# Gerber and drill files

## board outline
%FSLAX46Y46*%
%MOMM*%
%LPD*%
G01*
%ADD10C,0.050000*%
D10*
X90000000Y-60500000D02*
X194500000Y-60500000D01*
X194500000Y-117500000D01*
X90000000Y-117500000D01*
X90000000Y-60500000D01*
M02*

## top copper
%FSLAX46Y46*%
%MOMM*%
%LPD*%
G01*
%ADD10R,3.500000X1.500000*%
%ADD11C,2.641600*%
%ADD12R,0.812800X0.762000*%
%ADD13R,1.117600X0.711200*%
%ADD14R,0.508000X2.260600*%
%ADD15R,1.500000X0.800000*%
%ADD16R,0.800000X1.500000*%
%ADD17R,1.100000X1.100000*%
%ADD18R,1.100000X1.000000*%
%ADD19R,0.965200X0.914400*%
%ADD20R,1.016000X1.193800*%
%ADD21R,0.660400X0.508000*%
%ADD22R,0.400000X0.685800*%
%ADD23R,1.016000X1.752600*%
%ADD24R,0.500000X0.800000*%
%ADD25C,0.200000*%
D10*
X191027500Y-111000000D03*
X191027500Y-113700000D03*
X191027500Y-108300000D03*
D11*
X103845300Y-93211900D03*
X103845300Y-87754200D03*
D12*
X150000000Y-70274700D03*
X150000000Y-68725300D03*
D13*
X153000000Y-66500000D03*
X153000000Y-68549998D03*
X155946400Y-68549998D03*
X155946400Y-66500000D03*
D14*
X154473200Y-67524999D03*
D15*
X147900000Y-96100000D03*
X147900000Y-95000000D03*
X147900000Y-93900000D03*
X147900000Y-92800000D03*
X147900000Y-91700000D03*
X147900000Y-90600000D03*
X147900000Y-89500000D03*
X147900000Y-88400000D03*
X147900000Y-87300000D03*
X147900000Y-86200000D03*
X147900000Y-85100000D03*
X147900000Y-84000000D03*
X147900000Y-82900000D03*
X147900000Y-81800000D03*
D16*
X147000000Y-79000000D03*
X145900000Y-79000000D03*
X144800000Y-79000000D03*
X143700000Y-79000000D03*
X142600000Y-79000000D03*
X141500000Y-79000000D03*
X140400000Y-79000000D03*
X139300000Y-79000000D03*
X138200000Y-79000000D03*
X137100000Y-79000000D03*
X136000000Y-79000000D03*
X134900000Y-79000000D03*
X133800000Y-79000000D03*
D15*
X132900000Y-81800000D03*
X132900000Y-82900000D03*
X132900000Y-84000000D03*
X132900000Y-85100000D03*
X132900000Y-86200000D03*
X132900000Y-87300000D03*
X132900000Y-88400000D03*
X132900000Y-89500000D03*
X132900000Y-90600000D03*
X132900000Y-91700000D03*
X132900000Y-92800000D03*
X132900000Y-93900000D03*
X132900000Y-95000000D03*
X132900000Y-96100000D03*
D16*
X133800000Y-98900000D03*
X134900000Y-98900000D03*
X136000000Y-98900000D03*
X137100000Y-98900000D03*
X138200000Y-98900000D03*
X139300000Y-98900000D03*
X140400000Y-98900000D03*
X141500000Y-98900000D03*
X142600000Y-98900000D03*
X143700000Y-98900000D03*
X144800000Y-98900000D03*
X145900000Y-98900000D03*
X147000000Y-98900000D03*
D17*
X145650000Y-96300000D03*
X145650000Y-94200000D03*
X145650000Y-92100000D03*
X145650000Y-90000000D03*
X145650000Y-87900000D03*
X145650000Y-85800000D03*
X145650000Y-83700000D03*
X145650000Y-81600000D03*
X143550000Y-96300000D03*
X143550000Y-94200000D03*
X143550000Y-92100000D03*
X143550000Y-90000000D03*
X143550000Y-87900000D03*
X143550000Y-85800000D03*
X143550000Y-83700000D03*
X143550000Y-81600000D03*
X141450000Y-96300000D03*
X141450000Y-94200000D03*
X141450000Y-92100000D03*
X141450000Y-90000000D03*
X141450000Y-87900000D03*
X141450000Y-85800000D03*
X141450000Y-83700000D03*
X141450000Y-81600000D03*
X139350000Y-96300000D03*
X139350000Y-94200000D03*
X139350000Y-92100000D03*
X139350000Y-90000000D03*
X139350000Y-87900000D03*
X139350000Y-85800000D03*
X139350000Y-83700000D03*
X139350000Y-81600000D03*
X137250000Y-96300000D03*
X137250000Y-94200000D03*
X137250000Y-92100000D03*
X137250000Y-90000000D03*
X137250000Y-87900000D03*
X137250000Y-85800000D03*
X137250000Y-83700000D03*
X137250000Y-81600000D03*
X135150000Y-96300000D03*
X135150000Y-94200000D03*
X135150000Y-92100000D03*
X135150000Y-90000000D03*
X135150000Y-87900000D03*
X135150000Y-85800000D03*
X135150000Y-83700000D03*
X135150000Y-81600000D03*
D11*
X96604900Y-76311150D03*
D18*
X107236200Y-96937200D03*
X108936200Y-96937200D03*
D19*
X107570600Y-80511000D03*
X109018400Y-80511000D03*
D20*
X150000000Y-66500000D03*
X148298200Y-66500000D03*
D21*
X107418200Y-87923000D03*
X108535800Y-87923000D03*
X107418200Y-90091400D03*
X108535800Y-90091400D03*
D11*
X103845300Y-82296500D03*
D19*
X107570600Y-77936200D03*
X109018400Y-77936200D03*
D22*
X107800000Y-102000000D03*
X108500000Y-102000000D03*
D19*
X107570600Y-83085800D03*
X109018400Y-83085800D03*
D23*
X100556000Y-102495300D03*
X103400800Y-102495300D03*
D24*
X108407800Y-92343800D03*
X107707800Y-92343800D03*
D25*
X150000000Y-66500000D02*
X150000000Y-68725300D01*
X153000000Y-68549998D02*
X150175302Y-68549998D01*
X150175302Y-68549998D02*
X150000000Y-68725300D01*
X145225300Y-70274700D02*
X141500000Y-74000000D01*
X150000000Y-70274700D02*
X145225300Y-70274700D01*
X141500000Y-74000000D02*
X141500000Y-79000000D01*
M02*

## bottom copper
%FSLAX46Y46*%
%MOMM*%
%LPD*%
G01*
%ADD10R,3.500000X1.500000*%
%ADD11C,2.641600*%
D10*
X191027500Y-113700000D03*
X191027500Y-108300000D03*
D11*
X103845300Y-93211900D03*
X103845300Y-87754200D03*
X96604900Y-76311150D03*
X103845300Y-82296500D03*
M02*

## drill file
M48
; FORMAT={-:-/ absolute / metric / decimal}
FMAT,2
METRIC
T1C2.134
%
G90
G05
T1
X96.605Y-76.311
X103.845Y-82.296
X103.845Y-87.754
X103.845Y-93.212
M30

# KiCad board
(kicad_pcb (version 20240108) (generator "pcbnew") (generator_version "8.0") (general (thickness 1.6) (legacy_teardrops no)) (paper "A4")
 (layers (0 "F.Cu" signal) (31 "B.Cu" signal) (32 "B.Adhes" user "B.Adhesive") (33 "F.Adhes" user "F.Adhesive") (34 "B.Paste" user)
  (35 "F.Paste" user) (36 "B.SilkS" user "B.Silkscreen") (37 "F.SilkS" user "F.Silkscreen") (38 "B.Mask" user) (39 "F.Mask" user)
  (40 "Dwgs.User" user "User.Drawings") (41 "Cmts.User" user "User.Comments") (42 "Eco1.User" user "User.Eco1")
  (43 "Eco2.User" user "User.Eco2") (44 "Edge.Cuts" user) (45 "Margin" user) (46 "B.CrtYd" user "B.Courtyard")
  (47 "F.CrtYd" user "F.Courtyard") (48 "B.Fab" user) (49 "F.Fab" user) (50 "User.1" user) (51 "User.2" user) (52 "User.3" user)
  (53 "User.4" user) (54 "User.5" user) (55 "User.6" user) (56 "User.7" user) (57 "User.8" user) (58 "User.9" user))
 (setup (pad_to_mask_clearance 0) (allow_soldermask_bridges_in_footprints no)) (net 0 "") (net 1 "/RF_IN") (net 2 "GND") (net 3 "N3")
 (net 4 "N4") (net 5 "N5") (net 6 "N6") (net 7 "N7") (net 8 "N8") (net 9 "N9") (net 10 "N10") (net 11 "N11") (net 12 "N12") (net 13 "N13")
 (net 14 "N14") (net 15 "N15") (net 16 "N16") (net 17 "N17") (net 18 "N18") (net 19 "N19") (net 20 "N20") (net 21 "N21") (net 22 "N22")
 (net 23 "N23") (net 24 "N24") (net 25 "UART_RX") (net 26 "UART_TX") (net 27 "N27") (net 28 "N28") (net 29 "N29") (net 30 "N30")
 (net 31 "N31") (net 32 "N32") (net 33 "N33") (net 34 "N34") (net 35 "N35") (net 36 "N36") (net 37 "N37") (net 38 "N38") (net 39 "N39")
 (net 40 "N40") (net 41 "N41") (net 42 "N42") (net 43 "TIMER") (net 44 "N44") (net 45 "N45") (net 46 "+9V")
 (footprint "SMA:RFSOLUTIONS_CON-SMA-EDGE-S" (layer "F.Cu") (at 191.0275 111 180)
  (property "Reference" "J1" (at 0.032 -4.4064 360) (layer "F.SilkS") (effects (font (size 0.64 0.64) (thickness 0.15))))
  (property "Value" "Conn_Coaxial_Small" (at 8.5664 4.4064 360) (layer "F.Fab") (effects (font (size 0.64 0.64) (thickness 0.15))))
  (pad "1" smd rect (at 0 0 180) (size 3.5 1.5) (layers "F.Cu" "F.Paste" "F.Mask") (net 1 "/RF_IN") (solder_mask_margin 0.102))
  (pad "G1" smd rect (at 0 -2.7 180) (size 3.5 1.5) (layers "F.Cu" "F.Paste" "F.Mask") (solder_mask_margin 0.102))
  (pad "G2" smd rect (at 0 2.7 180) (size 3.5 1.5) (layers "F.Cu" "F.Paste" "F.Mask") (solder_mask_margin 0.102))
  (pad "G3" smd rect (at 0 -2.7 180) (size 3.5 1.5) (layers "B.Cu" "B.Paste" "B.Mask") (solder_mask_margin 0.102))
  (pad "G4" smd rect (at 0 2.7 180) (size 3.5 1.5) (layers "B.Cu" "B.Paste" "B.Mask") (solder_mask_margin 0.102)))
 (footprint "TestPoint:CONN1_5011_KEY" (layer "F.Cu") (at 103.8453 93.2119)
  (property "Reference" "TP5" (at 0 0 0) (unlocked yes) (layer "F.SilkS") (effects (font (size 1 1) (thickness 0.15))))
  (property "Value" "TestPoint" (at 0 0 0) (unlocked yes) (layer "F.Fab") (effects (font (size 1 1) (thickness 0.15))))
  (pad "1" thru_hole circle (at 0 0) (size 2.6416 2.6416) (drill 2.1336) (layers "*.Cu" "*.Mask") (remove_unused_layers no) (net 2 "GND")))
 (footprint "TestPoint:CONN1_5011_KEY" (layer "F.Cu") (at 103.8453 87.7542)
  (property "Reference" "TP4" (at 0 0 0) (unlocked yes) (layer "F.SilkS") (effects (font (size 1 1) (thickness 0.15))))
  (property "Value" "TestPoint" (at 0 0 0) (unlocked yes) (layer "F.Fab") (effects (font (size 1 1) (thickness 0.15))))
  (pad "1" thru_hole circle (at 0 0) (size 2.6416 2.6416) (drill 2.1336) (layers "*.Cu" "*.Mask") (remove_unused_layers no) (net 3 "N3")))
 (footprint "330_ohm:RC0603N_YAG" (layer "F.Cu") (at 150 69.5 90)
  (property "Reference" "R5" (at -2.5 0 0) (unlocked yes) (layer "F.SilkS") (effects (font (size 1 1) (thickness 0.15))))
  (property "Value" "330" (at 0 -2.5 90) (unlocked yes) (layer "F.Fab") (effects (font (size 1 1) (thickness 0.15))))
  (pad "1" smd rect (at -0.7747 0 90) (size 0.762 0.8128) (layers "F.Cu" "F.Paste" "F.Mask") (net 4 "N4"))
  (pad "2" smd rect (at 0.7747 0 90) (size 0.762 0.8128) (layers "F.Cu" "F.Paste" "F.Mask") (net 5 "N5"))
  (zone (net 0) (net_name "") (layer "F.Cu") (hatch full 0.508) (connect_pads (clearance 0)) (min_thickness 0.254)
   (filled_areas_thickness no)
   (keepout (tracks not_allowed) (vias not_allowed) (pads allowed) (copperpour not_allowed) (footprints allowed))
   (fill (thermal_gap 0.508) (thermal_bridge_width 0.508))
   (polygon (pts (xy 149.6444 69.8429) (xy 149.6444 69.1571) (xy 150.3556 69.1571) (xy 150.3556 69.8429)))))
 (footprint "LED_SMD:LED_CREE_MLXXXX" (layer "F.Cu") (at 154.4732 67.524999)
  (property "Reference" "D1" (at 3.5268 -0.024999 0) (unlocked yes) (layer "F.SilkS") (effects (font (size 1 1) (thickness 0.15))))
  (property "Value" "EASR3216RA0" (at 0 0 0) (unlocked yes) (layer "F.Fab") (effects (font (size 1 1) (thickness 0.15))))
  (pad "1" smd rect (at -1.4732 -1.024999) (size 1.1176 0.7112) (layers "F.Cu" "F.Paste" "F.Mask") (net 2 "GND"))
  (pad "2" smd rect (at -1.4732 1.024999) (size 1.1176 0.7112) (layers "F.Cu" "F.Paste" "F.Mask") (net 5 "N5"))
  (pad "3" smd rect (at 1.4732 1.024999) (size 1.1176 0.7112) (layers "F.Cu" "F.Paste" "F.Mask"))
  (pad "4" smd rect (at 1.4732 -1.024999) (size 1.1176 0.7112) (layers "F.Cu" "F.Paste" "F.Mask"))
  (pad "5" smd rect (at 0 0) (size 0.508 2.2606) (layers "F.Cu" "F.Paste" "F.Mask")))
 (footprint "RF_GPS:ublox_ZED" (layer "F.Cu") (at 140.4 88.95 180)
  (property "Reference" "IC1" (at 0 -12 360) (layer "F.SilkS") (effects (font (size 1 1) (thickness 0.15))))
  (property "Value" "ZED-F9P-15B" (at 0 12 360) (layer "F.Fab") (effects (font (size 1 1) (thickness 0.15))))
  (pad "1" smd rect (at -7.5 -7.15 180) (size 1.5 0.8) (layers "F.Cu" "F.Paste" "F.Mask") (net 2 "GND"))
  (pad "2" smd rect (at -7.5 -6.05 180) (size 1.5 0.8) (layers "F.Cu" "F.Paste" "F.Mask") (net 1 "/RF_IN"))
  (pad "3" smd rect (at -7.5 -4.95 180) (size 1.5 0.8) (layers "F.Cu" "F.Paste" "F.Mask") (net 2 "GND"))
  (pad "4" smd rect (at -7.5 -3.85 180) (size 1.5 0.8) (layers "F.Cu" "F.Paste" "F.Mask") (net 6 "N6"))
  (pad "5" smd rect (at -7.5 -2.75 180) (size 1.5 0.8) (layers "F.Cu" "F.Paste" "F.Mask") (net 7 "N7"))
  (pad "6" smd rect (at -7.5 -1.65 180) (size 1.5 0.8) (layers "F.Cu" "F.Paste" "F.Mask") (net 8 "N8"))
  (pad "7" smd rect (at -7.5 -0.55 180) (size 1.5 0.8) (layers "F.Cu" "F.Paste" "F.Mask") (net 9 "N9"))
  (pad "8" smd rect (at -7.5 0.55 180) (size 1.5 0.8) (layers "F.Cu" "F.Paste" "F.Mask") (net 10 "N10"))
  (pad "9" smd rect (at -7.5 1.65 180) (size 1.5 0.8) (layers "F.Cu" "F.Paste" "F.Mask") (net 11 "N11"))
  (pad "10" smd rect (at -7.5 2.75 180) (size 1.5 0.8) (layers "F.Cu" "F.Paste" "F.Mask") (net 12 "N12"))
  (pad "11" smd rect (at -7.5 3.85 180) (size 1.5 0.8) (layers "F.Cu" "F.Paste" "F.Mask") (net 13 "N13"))
  (pad "12" smd rect (at -7.5 4.95 180) (size 1.5 0.8) (layers "F.Cu" "F.Paste" "F.Mask") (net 2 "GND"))
  (pad "13" smd rect (at -7.5 6.05 180) (size 1.5 0.8) (layers "F.Cu" "F.Paste" "F.Mask") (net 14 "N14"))
  (pad "14" smd rect (at -7.5 7.15 180) (size 1.5 0.8) (layers "F.Cu" "F.Paste" "F.Mask") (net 2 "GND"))
  (pad "15" smd rect (at -6.6 9.95 270) (size 1.5 0.8) (layers "F.Cu" "F.Paste" "F.Mask") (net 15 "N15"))
  (pad "16" smd rect (at -5.5 9.95 270) (size 1.5 0.8) (layers "F.Cu" "F.Paste" "F.Mask") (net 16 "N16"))
  (pad "17" smd rect (at -4.4 9.95 270) (size 1.5 0.8) (layers "F.Cu" "F.Paste" "F.Mask") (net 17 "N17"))
  (pad "18" smd rect (at -3.3 9.95 90) (size 1.5 0.8) (layers "F.Cu" "F.Paste" "F.Mask") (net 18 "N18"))
  (pad "19" smd rect (at -2.2 9.95 270) (size 1.5 0.8) (layers "F.Cu" "F.Paste" "F.Mask") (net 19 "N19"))
  (pad "20" smd rect (at -1.1 9.95 270) (size 1.5 0.8) (layers "F.Cu" "F.Paste" "F.Mask") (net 4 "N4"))
  (pad "21" smd rect (at 0 9.95 270) (size 1.5 0.8) (layers "F.Cu" "F.Paste" "F.Mask") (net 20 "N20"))
  (pad "22" smd rect (at 1.1 9.95 270) (size 1.5 0.8) (layers "F.Cu" "F.Paste" "F.Mask") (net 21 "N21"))
  (pad "23" smd rect (at 2.2 9.95 270) (size 1.5 0.8) (layers "F.Cu" "F.Paste" "F.Mask") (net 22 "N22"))
  (pad "24" smd rect (at 3.3 9.95 270) (size 1.5 0.8) (layers "F.Cu" "F.Paste" "F.Mask") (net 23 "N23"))
  (pad "25" smd rect (at 4.4 9.95 270) (size 1.5 0.8) (layers "F.Cu" "F.Paste" "F.Mask") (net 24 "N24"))
  (pad "26" smd rect (at 5.5 9.95 270) (size 1.5 0.8) (layers "F.Cu" "F.Paste" "F.Mask") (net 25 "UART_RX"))
  (pad "27" smd rect (at 6.6 9.95 270) (size 1.5 0.8) (layers "F.Cu" "F.Paste" "F.Mask") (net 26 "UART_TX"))
  (pad "28" smd rect (at 7.5 7.15 180) (size 1.5 0.8) (layers "F.Cu" "F.Paste" "F.Mask") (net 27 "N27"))
  (pad "29" smd rect (at 7.5 6.05 180) (size 1.5 0.8) (layers "F.Cu" "F.Paste" "F.Mask") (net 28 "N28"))
  (pad "30" smd rect (at 7.5 4.95 180) (size 1.5 0.8) (layers "F.Cu" "F.Paste" "F.Mask") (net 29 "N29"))
  (pad "31" smd rect (at 7.5 3.85 180) (size 1.5 0.8) (layers "F.Cu" "F.Paste" "F.Mask") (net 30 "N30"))
  (pad "32" smd rect (at 7.5 2.75 180) (size 1.5 0.8) (layers "F.Cu" "F.Paste" "F.Mask") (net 2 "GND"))
  (pad "33" smd rect (at 7.5 1.65 180) (size 1.5 0.8) (layers "F.Cu" "F.Paste" "F.Mask") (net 3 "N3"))
  (pad "34" smd rect (at 7.5 0.55 180) (size 1.5 0.8) (layers "F.Cu" "F.Paste" "F.Mask") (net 3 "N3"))
  (pad "35" smd rect (at 7.5 -0.55 180) (size 1.5 0.8) (layers "F.Cu" "F.Paste" "F.Mask") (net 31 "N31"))
  (pad "36" smd rect (at 7.5 -1.65 180) (size 1.5 0.8) (layers "F.Cu" "F.Paste" "F.Mask") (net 2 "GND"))
  (pad "37" smd rect (at 7.5 -2.75 180) (size 1.5 0.8) (layers "F.Cu" "F.Paste" "F.Mask") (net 2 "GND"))
  (pad "38" smd rect (at 7.5 -3.85 180) (size 1.5 0.8) (layers "F.Cu" "F.Paste" "F.Mask") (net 2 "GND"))
  (pad "39" smd rect (at 7.5 -4.95 180) (size 1.5 0.8) (layers "F.Cu" "F.Paste" "F.Mask") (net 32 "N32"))
  (pad "40" smd rect (at 7.5 -6.05 180) (size 1.5 0.8) (layers "F.Cu" "F.Paste" "F.Mask") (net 32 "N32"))
  (pad "41" smd rect (at 7.5 -7.15 180) (size 1.5 0.8) (layers "F.Cu" "F.Paste" "F.Mask") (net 2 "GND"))
  (pad "42" smd rect (at 6.6 -9.95 270) (size 1.5 0.8) (layers "F.Cu" "F.Paste" "F.Mask") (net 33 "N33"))
  (pad "43" smd rect (at 5.5 -9.95 270) (size 1.5 0.8) (layers "F.Cu" "F.Paste" "F.Mask") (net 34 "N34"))
  (pad "44" smd rect (at 4.4 -9.95 270) (size 1.5 0.8) (layers "F.Cu" "F.Paste" "F.Mask") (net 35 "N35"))
  (pad "45" smd rect (at 3.3 -9.95 270) (size 1.5 0.8) (layers "F.Cu" "F.Paste" "F.Mask") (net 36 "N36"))
  (pad "46" smd rect (at 2.2 -9.95 270) (size 1.5 0.8) (layers "F.Cu" "F.Paste" "F.Mask") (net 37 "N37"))
  (pad "47" smd rect (at 1.1 -9.95 270) (size 1.5 0.8) (layers "F.Cu" "F.Paste" "F.Mask") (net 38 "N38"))
  (pad "48" smd rect (at 0 -9.95 270) (size 1.5 0.8) (layers "F.Cu" "F.Paste" "F.Mask") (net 2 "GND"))
  (pad "49" smd rect (at -1.1 -9.95 270) (size 1.5 0.8) (layers "F.Cu" "F.Paste" "F.Mask") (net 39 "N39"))
  (pad "50" smd rect (at -2.2 -9.95 270) (size 1.5 0.8) (layers "F.Cu" "F.Paste" "F.Mask") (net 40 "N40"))
  (pad "51" smd rect (at -3.3 -9.95 270) (size 1.5 0.8) (layers "F.Cu" "F.Paste" "F.Mask") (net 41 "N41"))
  (pad "52" smd rect (at -4.4 -9.95 270) (size 1.5 0.8) (layers "F.Cu" "F.Paste" "F.Mask") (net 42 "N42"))
  (pad "53" smd rect (at -5.5 -9.95 270) (size 1.5 0.8) (layers "F.Cu" "F.Paste" "F.Mask") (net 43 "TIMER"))
  (pad "54" smd rect (at -6.6 -9.95 270) (size 1.5 0.8) (layers "F.Cu" "F.Paste" "F.Mask") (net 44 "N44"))
  (pad "55" smd rect (at -5.25 -7.35 180) (size 1.1 1.1) (layers "F.Cu" "F.Paste" "F.Mask") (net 2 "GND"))
  (pad "55" smd rect (at -5.25 -5.25 180) (size 1.1 1.1) (layers "F.Cu" "F.Paste" "F.Mask") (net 2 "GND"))
  (pad "55" smd rect (at -5.25 -3.15 180) (size 1.1 1.1) (layers "F.Cu" "F.Paste" "F.Mask") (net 2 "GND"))
  (pad "55" smd rect (at -5.25 -1.05 180) (size 1.1 1.1) (layers "F.Cu" "F.Paste" "F.Mask") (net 2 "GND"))
  (pad "55" smd rect (at -5.25 1.05 180) (size 1.1 1.1) (layers "F.Cu" "F.Paste" "F.Mask") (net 2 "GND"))
  (pad "55" smd rect (at -5.25 3.15 180) (size 1.1 1.1) (layers "F.Cu" "F.Paste" "F.Mask") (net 2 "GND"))
  (pad "55" smd rect (at -5.25 5.25 180) (size 1.1 1.1) (layers "F.Cu" "F.Paste" "F.Mask") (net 2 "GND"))
  (pad "55" smd rect (at -5.25 7.35 180) (size 1.1 1.1) (layers "F.Cu" "F.Paste" "F.Mask") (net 2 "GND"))
  (pad "55" smd rect (at -3.15 -7.35 180) (size 1.1 1.1) (layers "F.Cu" "F.Paste" "F.Mask") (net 2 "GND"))
  (pad "55" smd rect (at -3.15 -5.25 180) (size 1.1 1.1) (layers "F.Cu" "F.Paste" "F.Mask") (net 2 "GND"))
  (pad "55" smd rect (at -3.15 -3.15 180) (size 1.1 1.1) (layers "F.Cu" "F.Paste" "F.Mask") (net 2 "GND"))
  (pad "55" smd rect (at -3.15 -1.05 180) (size 1.1 1.1) (layers "F.Cu" "F.Paste" "F.Mask") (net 2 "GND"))
  (pad "55" smd rect (at -3.15 1.05 180) (size 1.1 1.1) (layers "F.Cu" "F.Paste" "F.Mask") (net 2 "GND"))
  (pad "55" smd rect (at -3.15 3.15 180) (size 1.1 1.1) (layers "F.Cu" "F.Paste" "F.Mask") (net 2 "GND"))
  (pad "55" smd rect (at -3.15 5.25 180) (size 1.1 1.1) (layers "F.Cu" "F.Paste" "F.Mask") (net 2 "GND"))
  (pad "55" smd rect (at -3.15 7.35 180) (size 1.1 1.1) (layers "F.Cu" "F.Paste" "F.Mask") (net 2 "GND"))
  (pad "55" smd rect (at -1.05 -7.35 180) (size 1.1 1.1) (layers "F.Cu" "F.Paste" "F.Mask") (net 2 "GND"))
  (pad "55" smd rect (at -1.05 -5.25 180) (size 1.1 1.1) (layers "F.Cu" "F.Paste" "F.Mask") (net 2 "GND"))
  (pad "55" smd rect (at -1.05 -3.15 180) (size 1.1 1.1) (layers "F.Cu" "F.Paste" "F.Mask") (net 2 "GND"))
  (pad "55" smd rect (at -1.05 -1.05 180) (size 1.1 1.1) (layers "F.Cu" "F.Paste" "F.Mask") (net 2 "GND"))
  (pad "55" smd rect (at -1.05 1.05 180) (size 1.1 1.1) (layers "F.Cu" "F.Paste" "F.Mask") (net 2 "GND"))
  (pad "55" smd rect (at -1.05 3.15 180) (size 1.1 1.1) (layers "F.Cu" "F.Paste" "F.Mask") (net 2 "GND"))
  (pad "55" smd rect (at -1.05 5.25 180) (size 1.1 1.1) (layers "F.Cu" "F.Paste" "F.Mask") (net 2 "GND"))
  (pad "55" smd rect (at -1.05 7.35 180) (size 1.1 1.1) (layers "F.Cu" "F.Paste" "F.Mask") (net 2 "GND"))
  (pad "55" smd rect (at 1.05 -7.35 180) (size 1.1 1.1) (layers "F.Cu" "F.Paste" "F.Mask") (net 2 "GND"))
  (pad "55" smd rect (at 1.05 -5.25 180) (size 1.1 1.1) (layers "F.Cu" "F.Paste" "F.Mask") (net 2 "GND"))
  (pad "55" smd rect (at 1.05 -3.15 180) (size 1.1 1.1) (layers "F.Cu" "F.Paste" "F.Mask") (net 2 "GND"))
  (pad "55" smd rect (at 1.05 -1.05 180) (size 1.1 1.1) (layers "F.Cu" "F.Paste" "F.Mask") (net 2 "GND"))
  (pad "55" smd rect (at 1.05 1.05 180) (size 1.1 1.1) (layers "F.Cu" "F.Paste" "F.Mask") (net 2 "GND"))
  (pad "55" smd rect (at 1.05 3.15 180) (size 1.1 1.1) (layers "F.Cu" "F.Paste" "F.Mask") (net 2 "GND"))
  (pad "55" smd rect (at 1.05 5.25 180) (size 1.1 1.1) (layers "F.Cu" "F.Paste" "F.Mask") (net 2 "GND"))
  (pad "55" smd rect (at 1.05 7.35 180) (size 1.1 1.1) (layers "F.Cu" "F.Paste" "F.Mask") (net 2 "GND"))
  (pad "55" smd rect (at 3.15 -7.35 180) (size 1.1 1.1) (layers "F.Cu" "F.Paste" "F.Mask") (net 2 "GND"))
  (pad "55" smd rect (at 3.15 -5.25 180) (size 1.1 1.1) (layers "F.Cu" "F.Paste" "F.Mask") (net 2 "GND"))
  (pad "55" smd rect (at 3.15 -3.15 180) (size 1.1 1.1) (layers "F.Cu" "F.Paste" "F.Mask") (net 2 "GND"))
  (pad "55" smd rect (at 3.15 -1.05 180) (size 1.1 1.1) (layers "F.Cu" "F.Paste" "F.Mask") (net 2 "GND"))
  (pad "55" smd rect (at 3.15 1.05 180) (size 1.1 1.1) (layers "F.Cu" "F.Paste" "F.Mask") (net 2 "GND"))
  (pad "55" smd rect (at 3.15 3.15 180) (size 1.1 1.1) (layers "F.Cu" "F.Paste" "F.Mask") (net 2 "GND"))
  (pad "55" smd rect (at 3.15 5.25 180) (size 1.1 1.1) (layers "F.Cu" "F.Paste" "F.Mask") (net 2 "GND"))
  (pad "55" smd rect (at 3.15 7.35 180) (size 1.1 1.1) (layers "F.Cu" "F.Paste" "F.Mask") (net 2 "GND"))
  (pad "55" smd rect (at 5.25 -7.35 180) (size 1.1 1.1) (layers "F.Cu" "F.Paste" "F.Mask") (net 2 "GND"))
  (pad "55" smd rect (at 5.25 -5.25 180) (size 1.1 1.1) (layers "F.Cu" "F.Paste" "F.Mask") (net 2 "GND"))
  (pad "55" smd rect (at 5.25 -3.15 180) (size 1.1 1.1) (layers "F.Cu" "F.Paste" "F.Mask") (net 2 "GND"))
  (pad "55" smd rect (at 5.25 -1.05 180) (size 1.1 1.1) (layers "F.Cu" "F.Paste" "F.Mask") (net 2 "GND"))
  (pad "55" smd rect (at 5.25 1.05 180) (size 1.1 1.1) (layers "F.Cu" "F.Paste" "F.Mask") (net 2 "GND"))
  (pad "55" smd rect (at 5.25 3.15 180) (size 1.1 1.1) (layers "F.Cu" "F.Paste" "F.Mask") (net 2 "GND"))
  (pad "55" smd rect (at 5.25 5.25 180) (size 1.1 1.1) (layers "F.Cu" "F.Paste" "F.Mask") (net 2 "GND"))
  (pad "55" smd rect (at 5.25 7.35 180) (size 1.1 1.1) (layers "F.Cu" "F.Paste" "F.Mask") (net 2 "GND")))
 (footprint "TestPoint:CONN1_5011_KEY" (layer "F.Cu") (at 96.6049 76.31115)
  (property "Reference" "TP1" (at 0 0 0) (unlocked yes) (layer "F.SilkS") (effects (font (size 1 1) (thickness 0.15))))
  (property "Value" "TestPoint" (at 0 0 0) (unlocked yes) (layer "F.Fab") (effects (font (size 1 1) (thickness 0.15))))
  (pad "1" thru_hole circle (at 0 0) (size 2.6416 2.6416) (drill 2.1336) (layers "*.Cu" "*.Mask") (remove_unused_layers no) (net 1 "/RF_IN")))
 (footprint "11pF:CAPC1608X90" (layer "F.Cu") (at 108.0862 96.9372)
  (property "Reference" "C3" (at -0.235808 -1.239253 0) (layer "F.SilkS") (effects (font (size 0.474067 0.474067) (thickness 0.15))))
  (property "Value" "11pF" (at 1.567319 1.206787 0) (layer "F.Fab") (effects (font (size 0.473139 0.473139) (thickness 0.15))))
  (pad "1" smd rect (at -0.85 0) (size 1.1 1) (layers "F.Cu" "F.Paste" "F.Mask") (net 1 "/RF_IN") (solder_mask_margin 0.102))
  (pad "2" smd rect (at 0.85 0) (size 1.1 1) (layers "F.Cu" "F.Paste" "F.Mask") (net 2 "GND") (solder_mask_margin 0.102)))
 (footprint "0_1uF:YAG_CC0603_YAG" (layer "F.Cu") (at 108.2945 80.511)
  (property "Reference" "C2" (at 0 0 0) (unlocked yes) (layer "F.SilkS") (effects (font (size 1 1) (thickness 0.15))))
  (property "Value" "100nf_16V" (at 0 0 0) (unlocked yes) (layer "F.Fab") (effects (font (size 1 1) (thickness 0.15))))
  (pad "1" smd rect (at -0.7239 0) (size 0.9652 0.9144) (layers "F.Cu" "F.Paste" "F.Mask") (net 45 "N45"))
  (pad "2" smd rect (at 0.7239 0) (size 0.9652 0.9144) (layers "F.Cu" "F.Paste" "F.Mask") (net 2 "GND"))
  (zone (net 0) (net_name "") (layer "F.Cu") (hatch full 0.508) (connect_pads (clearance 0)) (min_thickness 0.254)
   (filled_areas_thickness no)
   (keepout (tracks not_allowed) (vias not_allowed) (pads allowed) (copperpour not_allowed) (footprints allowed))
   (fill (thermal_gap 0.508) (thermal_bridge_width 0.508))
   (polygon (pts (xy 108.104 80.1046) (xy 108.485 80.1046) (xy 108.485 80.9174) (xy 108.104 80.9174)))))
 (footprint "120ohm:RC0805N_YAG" (layer "F.Cu") (at 149.1491 66.5 180)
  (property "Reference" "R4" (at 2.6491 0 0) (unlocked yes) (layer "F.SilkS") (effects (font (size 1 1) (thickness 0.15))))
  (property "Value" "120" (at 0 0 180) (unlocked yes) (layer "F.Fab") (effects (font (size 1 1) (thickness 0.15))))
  (pad "1" smd rect (at -0.8509 0 180) (size 1.016 1.1938) (layers "F.Cu" "F.Paste" "F.Mask") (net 5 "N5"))
  (pad "2" smd rect (at 0.8509 0 180) (size 1.016 1.1938) (layers "F.Cu" "F.Paste" "F.Mask") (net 2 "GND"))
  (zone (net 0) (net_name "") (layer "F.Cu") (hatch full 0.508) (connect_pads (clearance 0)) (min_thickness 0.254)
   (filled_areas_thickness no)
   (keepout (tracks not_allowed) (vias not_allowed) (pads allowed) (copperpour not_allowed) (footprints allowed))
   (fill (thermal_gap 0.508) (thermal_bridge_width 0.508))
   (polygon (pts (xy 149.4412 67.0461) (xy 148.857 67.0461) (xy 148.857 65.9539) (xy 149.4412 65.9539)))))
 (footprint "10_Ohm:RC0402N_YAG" (layer "F.Cu") (at 107.977 87.923)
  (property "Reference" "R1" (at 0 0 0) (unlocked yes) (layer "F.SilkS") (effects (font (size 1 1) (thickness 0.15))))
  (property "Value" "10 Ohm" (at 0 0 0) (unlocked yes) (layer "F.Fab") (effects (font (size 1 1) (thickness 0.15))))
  (pad "1" smd rect (at -0.5588 0) (size 0.6604 0.508) (layers "F.Cu" "F.Paste" "F.Mask") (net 3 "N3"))
  (pad "2" smd rect (at 0.5588 0) (size 0.6604 0.508) (layers "F.Cu" "F.Paste" "F.Mask") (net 45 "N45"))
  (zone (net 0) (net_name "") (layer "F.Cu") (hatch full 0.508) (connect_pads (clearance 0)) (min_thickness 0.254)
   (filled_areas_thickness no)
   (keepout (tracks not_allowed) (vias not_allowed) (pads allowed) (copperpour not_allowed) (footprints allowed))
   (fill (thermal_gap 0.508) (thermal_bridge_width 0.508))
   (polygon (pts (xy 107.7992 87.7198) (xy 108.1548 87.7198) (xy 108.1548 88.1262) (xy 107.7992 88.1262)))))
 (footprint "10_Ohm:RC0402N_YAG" (layer "F.Cu") (at 107.977 90.0914)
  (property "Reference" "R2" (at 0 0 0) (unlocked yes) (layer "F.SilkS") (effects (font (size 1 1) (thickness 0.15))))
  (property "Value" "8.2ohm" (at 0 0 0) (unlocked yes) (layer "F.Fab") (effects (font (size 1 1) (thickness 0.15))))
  (pad "1" smd rect (at -0.5588 0) (size 0.6604 0.508) (layers "F.Cu" "F.Paste" "F.Mask") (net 1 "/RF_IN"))
  (pad "2" smd rect (at 0.5588 0) (size 0.6604 0.508) (layers "F.Cu" "F.Paste" "F.Mask") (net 1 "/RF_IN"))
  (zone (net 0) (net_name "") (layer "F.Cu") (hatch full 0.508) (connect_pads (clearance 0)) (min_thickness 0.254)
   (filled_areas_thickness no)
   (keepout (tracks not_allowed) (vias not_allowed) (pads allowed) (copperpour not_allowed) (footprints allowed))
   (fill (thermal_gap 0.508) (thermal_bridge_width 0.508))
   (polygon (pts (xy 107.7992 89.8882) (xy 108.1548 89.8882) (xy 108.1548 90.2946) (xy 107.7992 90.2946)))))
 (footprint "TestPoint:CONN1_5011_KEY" (layer "F.Cu") (at 103.8453 82.2965)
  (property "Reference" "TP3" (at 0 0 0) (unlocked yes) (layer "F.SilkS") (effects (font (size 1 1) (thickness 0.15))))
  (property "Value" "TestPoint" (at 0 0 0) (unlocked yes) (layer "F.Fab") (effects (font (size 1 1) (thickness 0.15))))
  (pad "1" thru_hole circle (at 0 0) (size 2.6416 2.6416) (drill 2.1336) (layers "*.Cu" "*.Mask") (remove_unused_layers no) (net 1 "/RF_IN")))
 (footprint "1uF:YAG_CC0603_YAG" (layer "F.Cu") (at 108.2945 77.9362)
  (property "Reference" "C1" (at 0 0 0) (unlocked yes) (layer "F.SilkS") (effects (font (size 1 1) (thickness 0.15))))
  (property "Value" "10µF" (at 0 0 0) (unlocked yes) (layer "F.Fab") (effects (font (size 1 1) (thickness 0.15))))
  (pad "1" smd rect (at -0.7239 0) (size 0.9652 0.9144) (layers "F.Cu" "F.Paste" "F.Mask") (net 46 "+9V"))
  (pad "2" smd rect (at 0.7239 0) (size 0.9652 0.9144) (layers "F.Cu" "F.Paste" "F.Mask") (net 2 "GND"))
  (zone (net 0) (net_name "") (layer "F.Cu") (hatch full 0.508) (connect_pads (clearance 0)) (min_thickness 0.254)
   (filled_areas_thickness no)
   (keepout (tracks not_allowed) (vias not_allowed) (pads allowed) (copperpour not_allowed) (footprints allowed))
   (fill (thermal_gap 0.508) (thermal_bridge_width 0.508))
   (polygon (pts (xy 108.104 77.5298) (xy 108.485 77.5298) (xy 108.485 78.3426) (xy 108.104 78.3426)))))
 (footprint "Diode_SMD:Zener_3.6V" (layer "F.Cu") (at 108.15 102)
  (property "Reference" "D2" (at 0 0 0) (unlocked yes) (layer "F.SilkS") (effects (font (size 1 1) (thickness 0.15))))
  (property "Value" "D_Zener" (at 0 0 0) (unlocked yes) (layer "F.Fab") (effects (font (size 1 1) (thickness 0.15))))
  (pad "1" smd rect (at -0.35 0) (size 0.4 0.6858) (layers "F.Cu" "F.Paste" "F.Mask") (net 1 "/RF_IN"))
  (pad "2" smd rect (at 0.35 0) (size 0.4 0.6858) (layers "F.Cu" "F.Paste" "F.Mask") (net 2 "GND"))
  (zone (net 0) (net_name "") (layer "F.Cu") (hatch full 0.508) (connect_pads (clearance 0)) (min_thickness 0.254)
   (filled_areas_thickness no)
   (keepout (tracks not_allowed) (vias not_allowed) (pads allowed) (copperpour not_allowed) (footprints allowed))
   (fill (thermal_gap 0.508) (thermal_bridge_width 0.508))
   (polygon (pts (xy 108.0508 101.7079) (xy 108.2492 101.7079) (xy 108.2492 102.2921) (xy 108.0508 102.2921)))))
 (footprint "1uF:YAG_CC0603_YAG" (layer "F.Cu") (at 108.2945 83.0858)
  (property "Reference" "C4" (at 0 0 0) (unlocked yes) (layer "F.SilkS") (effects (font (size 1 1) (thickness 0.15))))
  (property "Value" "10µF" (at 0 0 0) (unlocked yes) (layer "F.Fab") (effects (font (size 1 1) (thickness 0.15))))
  (pad "1" smd rect (at -0.7239 0) (size 0.9652 0.9144) (layers "F.Cu" "F.Paste" "F.Mask") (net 3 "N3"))
  (pad "2" smd rect (at 0.7239 0) (size 0.9652 0.9144) (layers "F.Cu" "F.Paste" "F.Mask") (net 2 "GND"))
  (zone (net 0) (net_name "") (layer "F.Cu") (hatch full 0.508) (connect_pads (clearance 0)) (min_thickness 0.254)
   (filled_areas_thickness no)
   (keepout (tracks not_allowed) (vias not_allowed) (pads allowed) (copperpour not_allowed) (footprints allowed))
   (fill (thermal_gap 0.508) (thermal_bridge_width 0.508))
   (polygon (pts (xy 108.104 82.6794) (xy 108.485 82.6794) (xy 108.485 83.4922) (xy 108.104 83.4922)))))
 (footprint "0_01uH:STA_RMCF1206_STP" (layer "F.Cu") (at 101.9784 102.4953)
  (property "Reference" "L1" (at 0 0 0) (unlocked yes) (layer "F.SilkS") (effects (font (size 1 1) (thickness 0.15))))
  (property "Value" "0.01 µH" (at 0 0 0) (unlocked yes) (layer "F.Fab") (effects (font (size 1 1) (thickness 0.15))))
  (pad "1" smd rect (at -1.4224 0) (size 1.016 1.7526) (layers "F.Cu" "F.Paste" "F.Mask") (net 1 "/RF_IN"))
  (pad "2" smd rect (at 1.4224 0) (size 1.016 1.7526) (layers "F.Cu" "F.Paste" "F.Mask") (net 45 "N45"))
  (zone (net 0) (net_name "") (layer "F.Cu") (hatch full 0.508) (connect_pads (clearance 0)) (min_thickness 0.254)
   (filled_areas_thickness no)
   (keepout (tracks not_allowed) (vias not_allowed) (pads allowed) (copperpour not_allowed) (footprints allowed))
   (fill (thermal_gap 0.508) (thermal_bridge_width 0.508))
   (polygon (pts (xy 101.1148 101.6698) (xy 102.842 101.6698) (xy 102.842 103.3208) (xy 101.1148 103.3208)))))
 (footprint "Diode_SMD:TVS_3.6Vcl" (layer "F.Cu") (at 108.0578 92.3438)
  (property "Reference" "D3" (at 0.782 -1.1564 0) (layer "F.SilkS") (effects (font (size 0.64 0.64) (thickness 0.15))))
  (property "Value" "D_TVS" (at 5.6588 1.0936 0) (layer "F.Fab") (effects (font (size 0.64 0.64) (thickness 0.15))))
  (pad "A" smd rect (at 0.35 0) (size 0.5 0.8) (layers "F.Cu"))
  (pad "K" smd rect (at -0.35 0) (size 0.5 0.8) (layers "F.Cu")))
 (gr_rect (start 90 60.5) (end 194.5 117.5) (stroke (width 0.05) (type default)) (fill none) (layer "Edge.Cuts"))
 (segment (start 150 66.5) (end 150 68.7253) (width 0.2) (layer "F.Cu") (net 5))
 (segment (start 153 68.549998) (end 150.175302 68.549998) (width 0.2) (layer "F.Cu") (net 5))
 (segment (start 150.175302 68.549998) (end 150 68.7253) (width 0.2) (layer "F.Cu") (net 5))
 (segment (start 145.2253 70.2747) (end 141.5 74) (width 0.2) (layer "F.Cu") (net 4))
 (segment (start 150 70.2747) (end 145.2253 70.2747) (width 0.2) (layer "F.Cu") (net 4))
 (segment (start 141.5 74) (end 141.5 79) (width 0.2) (layer "F.Cu") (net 4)))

